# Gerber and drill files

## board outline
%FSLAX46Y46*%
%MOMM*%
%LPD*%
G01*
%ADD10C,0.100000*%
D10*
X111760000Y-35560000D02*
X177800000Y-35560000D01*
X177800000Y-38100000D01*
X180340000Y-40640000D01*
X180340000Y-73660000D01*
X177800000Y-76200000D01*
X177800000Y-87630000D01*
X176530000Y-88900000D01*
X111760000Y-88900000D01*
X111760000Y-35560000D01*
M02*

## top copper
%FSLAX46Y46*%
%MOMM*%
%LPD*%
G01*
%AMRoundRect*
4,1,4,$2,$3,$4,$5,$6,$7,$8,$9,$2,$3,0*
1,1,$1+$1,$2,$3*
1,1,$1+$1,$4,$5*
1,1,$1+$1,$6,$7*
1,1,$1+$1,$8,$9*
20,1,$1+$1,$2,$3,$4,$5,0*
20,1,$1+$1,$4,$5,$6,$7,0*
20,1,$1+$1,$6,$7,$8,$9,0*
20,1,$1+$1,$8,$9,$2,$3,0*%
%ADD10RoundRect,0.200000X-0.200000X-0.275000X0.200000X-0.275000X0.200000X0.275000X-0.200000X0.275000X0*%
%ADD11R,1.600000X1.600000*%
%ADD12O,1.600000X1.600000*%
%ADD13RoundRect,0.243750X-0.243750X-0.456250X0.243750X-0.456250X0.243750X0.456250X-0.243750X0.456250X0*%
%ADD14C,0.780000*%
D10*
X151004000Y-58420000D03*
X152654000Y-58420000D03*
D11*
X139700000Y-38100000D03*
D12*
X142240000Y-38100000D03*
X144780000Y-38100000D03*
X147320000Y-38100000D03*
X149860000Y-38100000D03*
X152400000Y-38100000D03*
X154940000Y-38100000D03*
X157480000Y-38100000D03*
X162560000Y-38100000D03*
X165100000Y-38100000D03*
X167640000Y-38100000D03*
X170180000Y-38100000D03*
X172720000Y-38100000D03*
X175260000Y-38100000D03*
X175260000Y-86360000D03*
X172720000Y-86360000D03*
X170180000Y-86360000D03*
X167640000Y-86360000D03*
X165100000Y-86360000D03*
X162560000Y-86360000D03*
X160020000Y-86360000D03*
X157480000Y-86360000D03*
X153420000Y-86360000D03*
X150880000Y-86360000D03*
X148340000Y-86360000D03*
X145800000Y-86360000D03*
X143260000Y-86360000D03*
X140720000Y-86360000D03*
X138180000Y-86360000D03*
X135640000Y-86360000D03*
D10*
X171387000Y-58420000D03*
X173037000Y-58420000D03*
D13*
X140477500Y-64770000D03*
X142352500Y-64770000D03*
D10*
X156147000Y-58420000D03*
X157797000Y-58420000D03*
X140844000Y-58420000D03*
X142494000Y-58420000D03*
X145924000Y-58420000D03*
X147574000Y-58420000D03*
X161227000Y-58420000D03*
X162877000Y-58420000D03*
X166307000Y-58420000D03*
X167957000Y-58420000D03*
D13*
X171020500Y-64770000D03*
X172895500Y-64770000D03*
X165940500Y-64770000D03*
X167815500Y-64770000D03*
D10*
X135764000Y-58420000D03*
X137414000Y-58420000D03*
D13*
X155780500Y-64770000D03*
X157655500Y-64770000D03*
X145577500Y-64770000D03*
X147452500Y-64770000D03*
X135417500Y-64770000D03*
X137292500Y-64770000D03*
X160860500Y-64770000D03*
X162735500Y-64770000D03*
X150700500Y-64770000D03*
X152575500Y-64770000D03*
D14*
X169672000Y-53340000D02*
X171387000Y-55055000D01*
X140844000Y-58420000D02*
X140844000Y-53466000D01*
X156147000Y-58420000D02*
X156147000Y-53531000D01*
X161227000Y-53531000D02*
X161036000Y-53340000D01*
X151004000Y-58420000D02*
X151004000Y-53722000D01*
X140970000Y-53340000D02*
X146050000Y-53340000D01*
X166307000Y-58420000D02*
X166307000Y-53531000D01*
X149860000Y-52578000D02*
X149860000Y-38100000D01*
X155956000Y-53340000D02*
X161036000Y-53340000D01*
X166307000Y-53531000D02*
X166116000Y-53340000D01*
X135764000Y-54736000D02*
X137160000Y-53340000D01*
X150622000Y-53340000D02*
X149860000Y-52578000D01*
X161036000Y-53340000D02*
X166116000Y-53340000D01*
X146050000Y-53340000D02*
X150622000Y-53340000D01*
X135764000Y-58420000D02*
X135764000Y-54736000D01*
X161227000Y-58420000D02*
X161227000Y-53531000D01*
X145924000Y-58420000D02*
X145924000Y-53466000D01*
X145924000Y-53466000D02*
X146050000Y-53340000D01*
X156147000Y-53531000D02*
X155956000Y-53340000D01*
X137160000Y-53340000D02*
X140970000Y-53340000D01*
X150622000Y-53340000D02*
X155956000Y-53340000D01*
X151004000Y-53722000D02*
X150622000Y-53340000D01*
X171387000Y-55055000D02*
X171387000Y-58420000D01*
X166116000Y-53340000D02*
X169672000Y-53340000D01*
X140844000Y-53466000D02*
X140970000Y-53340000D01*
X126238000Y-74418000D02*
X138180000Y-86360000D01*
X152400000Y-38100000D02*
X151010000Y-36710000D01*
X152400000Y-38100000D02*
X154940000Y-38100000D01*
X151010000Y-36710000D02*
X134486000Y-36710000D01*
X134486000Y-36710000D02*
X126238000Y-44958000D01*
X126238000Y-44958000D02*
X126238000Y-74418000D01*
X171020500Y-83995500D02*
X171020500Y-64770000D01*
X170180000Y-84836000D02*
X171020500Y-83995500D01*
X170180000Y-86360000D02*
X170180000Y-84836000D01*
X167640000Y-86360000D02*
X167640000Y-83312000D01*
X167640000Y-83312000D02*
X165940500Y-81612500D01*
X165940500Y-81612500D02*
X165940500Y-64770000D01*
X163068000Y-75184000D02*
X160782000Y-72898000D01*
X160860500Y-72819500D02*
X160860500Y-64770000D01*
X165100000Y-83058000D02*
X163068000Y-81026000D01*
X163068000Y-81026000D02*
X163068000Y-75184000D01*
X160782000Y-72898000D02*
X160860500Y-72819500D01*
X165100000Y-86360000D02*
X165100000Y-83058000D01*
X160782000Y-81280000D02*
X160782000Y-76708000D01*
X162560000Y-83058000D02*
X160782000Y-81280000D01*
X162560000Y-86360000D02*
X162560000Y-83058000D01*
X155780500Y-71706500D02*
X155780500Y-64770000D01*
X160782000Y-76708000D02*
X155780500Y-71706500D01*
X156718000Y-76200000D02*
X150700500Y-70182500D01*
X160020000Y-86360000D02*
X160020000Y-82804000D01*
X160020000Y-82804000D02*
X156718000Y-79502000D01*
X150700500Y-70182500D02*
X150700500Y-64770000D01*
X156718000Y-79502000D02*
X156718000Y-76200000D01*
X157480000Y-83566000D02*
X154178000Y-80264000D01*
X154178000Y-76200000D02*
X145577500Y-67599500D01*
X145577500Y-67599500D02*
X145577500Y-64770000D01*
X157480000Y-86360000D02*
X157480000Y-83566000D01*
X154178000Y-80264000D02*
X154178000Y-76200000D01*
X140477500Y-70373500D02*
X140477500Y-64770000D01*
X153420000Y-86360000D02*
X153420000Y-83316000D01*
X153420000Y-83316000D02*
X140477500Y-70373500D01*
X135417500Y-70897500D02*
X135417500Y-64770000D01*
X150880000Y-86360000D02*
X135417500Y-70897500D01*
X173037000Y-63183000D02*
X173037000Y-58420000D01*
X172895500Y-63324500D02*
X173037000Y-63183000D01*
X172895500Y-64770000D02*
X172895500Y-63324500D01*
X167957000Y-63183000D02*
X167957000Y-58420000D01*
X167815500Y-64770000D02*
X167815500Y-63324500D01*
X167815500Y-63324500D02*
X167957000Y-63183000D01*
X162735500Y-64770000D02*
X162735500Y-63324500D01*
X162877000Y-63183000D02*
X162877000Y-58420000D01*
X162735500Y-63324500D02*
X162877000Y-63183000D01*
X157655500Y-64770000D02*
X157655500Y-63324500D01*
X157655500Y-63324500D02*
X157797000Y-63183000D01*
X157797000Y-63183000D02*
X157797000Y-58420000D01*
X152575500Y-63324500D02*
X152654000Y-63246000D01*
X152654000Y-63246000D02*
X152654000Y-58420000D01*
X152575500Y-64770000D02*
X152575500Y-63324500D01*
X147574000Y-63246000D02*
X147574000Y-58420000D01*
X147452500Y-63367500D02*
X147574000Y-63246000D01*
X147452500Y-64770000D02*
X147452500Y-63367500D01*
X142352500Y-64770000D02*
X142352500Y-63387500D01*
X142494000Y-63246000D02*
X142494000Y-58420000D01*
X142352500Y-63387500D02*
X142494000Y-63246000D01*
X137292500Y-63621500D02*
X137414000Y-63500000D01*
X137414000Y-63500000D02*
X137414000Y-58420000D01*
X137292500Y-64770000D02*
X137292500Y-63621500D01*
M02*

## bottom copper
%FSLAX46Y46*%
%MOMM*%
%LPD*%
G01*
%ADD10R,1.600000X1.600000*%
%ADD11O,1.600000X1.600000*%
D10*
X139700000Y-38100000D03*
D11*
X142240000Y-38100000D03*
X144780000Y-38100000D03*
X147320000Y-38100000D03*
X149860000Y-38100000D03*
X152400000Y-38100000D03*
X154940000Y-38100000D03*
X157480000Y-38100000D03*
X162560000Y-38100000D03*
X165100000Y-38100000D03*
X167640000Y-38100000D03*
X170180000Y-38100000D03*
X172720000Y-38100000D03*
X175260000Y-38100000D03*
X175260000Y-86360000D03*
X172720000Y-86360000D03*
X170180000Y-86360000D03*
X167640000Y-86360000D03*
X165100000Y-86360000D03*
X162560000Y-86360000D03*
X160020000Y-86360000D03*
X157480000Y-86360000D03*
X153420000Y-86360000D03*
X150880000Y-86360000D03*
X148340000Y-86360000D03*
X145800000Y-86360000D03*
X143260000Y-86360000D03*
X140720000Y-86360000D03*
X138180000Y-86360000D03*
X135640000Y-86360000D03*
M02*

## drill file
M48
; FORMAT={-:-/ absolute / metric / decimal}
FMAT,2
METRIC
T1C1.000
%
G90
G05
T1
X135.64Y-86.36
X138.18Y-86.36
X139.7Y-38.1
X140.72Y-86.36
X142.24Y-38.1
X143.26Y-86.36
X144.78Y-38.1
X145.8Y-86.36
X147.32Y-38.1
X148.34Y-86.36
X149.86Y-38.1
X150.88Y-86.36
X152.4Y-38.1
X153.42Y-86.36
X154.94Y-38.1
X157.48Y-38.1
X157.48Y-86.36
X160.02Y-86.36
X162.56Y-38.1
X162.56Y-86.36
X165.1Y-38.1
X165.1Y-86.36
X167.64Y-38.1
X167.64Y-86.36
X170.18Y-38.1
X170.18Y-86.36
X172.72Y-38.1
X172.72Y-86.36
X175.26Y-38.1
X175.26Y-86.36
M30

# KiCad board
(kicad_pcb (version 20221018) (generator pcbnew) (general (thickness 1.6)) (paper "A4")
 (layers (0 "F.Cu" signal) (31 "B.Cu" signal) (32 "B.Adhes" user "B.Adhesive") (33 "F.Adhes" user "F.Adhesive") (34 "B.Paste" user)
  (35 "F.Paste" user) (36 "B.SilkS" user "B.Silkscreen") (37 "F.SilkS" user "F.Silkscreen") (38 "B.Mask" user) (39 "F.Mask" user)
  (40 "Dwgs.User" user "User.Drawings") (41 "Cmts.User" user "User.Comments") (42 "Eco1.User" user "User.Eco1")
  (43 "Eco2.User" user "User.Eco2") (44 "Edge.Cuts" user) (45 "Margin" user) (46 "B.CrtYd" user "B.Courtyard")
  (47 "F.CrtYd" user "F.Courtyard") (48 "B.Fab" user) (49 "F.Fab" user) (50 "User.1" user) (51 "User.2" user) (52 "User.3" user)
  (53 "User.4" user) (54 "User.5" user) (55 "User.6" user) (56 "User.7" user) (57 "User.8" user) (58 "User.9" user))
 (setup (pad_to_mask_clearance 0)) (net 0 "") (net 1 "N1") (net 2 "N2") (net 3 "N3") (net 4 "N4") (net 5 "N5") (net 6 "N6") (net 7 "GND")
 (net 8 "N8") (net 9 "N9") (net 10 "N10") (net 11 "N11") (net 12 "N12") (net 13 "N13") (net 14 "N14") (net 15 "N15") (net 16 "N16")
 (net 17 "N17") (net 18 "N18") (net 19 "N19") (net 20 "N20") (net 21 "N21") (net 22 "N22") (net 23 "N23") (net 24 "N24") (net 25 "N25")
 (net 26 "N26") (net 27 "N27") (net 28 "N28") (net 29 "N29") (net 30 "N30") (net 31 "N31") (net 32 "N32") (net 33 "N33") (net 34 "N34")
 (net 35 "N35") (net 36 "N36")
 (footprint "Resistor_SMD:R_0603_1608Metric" (layer "F.Cu") (at 151.829 58.42)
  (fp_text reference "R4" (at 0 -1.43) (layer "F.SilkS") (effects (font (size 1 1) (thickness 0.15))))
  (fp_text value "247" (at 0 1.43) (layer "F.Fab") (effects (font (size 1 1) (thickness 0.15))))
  (pad "1" smd roundrect (at -0.825 0) (size 0.8 0.95) (layers "F.Cu" "F.Paste" "F.Mask") (roundrect_rratio 0.25) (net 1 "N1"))
  (pad "2" smd roundrect (at 0.825 0) (size 0.8 0.95) (layers "F.Cu" "F.Paste" "F.Mask") (roundrect_rratio 0.25) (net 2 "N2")))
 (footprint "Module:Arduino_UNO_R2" (layer "F.Cu") (at 139.7 38.1)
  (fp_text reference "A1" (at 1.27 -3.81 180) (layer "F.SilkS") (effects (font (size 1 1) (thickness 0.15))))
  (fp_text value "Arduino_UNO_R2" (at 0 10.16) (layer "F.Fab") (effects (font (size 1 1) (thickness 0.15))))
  (pad "1" thru_hole rect (at 0 0 90) (size 1.6 1.6) (drill 1) (layers "*.Cu" "*.Mask") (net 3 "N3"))
  (pad "2" thru_hole oval (at 2.54 0 90) (size 1.6 1.6) (drill 1) (layers "*.Cu" "*.Mask") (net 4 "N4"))
  (pad "3" thru_hole oval (at 5.08 0 90) (size 1.6 1.6) (drill 1) (layers "*.Cu" "*.Mask") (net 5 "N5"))
  (pad "4" thru_hole oval (at 7.62 0 90) (size 1.6 1.6) (drill 1) (layers "*.Cu" "*.Mask") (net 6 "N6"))
  (pad "5" thru_hole oval (at 10.16 0 90) (size 1.6 1.6) (drill 1) (layers "*.Cu" "*.Mask") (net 1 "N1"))
  (pad "6" thru_hole oval (at 12.7 0 90) (size 1.6 1.6) (drill 1) (layers "*.Cu" "*.Mask") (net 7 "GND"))
  (pad "7" thru_hole oval (at 15.24 0 90) (size 1.6 1.6) (drill 1) (layers "*.Cu" "*.Mask") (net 7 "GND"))
  (pad "8" thru_hole oval (at 17.78 0 90) (size 1.6 1.6) (drill 1) (layers "*.Cu" "*.Mask") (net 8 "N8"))
  (pad "9" thru_hole oval (at 22.86 0 90) (size 1.6 1.6) (drill 1) (layers "*.Cu" "*.Mask") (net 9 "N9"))
  (pad "10" thru_hole oval (at 25.4 0 90) (size 1.6 1.6) (drill 1) (layers "*.Cu" "*.Mask") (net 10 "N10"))
  (pad "11" thru_hole oval (at 27.94 0 90) (size 1.6 1.6) (drill 1) (layers "*.Cu" "*.Mask") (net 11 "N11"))
  (pad "12" thru_hole oval (at 30.48 0 90) (size 1.6 1.6) (drill 1) (layers "*.Cu" "*.Mask") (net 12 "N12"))
  (pad "13" thru_hole oval (at 33.02 0 90) (size 1.6 1.6) (drill 1) (layers "*.Cu" "*.Mask") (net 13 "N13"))
  (pad "14" thru_hole oval (at 35.56 0 90) (size 1.6 1.6) (drill 1) (layers "*.Cu" "*.Mask") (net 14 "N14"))
  (pad "15" thru_hole oval (at 35.56 48.26 90) (size 1.6 1.6) (drill 1) (layers "*.Cu" "*.Mask") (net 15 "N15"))
  (pad "16" thru_hole oval (at 33.02 48.26 90) (size 1.6 1.6) (drill 1) (layers "*.Cu" "*.Mask") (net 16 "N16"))
  (pad "17" thru_hole oval (at 30.48 48.26 90) (size 1.6 1.6) (drill 1) (layers "*.Cu" "*.Mask") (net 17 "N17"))
  (pad "18" thru_hole oval (at 27.94 48.26 90) (size 1.6 1.6) (drill 1) (layers "*.Cu" "*.Mask") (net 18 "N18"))
  (pad "19" thru_hole oval (at 25.4 48.26 90) (size 1.6 1.6) (drill 1) (layers "*.Cu" "*.Mask") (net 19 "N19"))
  (pad "20" thru_hole oval (at 22.86 48.26 90) (size 1.6 1.6) (drill 1) (layers "*.Cu" "*.Mask") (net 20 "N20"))
  (pad "21" thru_hole oval (at 20.32 48.26 90) (size 1.6 1.6) (drill 1) (layers "*.Cu" "*.Mask") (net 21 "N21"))
  (pad "22" thru_hole oval (at 17.78 48.26 90) (size 1.6 1.6) (drill 1) (layers "*.Cu" "*.Mask") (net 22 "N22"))
  (pad "23" thru_hole oval (at 13.72 48.26 90) (size 1.6 1.6) (drill 1) (layers "*.Cu" "*.Mask") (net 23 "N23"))
  (pad "24" thru_hole oval (at 11.18 48.26 90) (size 1.6 1.6) (drill 1) (layers "*.Cu" "*.Mask") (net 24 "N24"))
  (pad "25" thru_hole oval (at 8.64 48.26 90) (size 1.6 1.6) (drill 1) (layers "*.Cu" "*.Mask") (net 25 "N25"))
  (pad "26" thru_hole oval (at 6.1 48.26 90) (size 1.6 1.6) (drill 1) (layers "*.Cu" "*.Mask") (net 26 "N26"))
  (pad "27" thru_hole oval (at 3.56 48.26 90) (size 1.6 1.6) (drill 1) (layers "*.Cu" "*.Mask") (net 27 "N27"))
  (pad "28" thru_hole oval (at 1.02 48.26 90) (size 1.6 1.6) (drill 1) (layers "*.Cu" "*.Mask") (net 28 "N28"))
  (pad "29" thru_hole oval (at -1.52 48.26 90) (size 1.6 1.6) (drill 1) (layers "*.Cu" "*.Mask") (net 7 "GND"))
  (pad "30" thru_hole oval (at -4.06 48.26 90) (size 1.6 1.6) (drill 1) (layers "*.Cu" "*.Mask") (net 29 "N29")))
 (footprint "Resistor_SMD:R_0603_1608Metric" (layer "F.Cu") (at 172.212 58.42)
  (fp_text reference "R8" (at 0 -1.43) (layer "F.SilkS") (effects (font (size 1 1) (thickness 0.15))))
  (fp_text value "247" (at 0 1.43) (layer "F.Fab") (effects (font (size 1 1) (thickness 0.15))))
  (pad "1" smd roundrect (at -0.825 0) (size 0.8 0.95) (layers "F.Cu" "F.Paste" "F.Mask") (roundrect_rratio 0.25) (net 1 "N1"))
  (pad "2" smd roundrect (at 0.825 0) (size 0.8 0.95) (layers "F.Cu" "F.Paste" "F.Mask") (roundrect_rratio 0.25) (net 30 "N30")))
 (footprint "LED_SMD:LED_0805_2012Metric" (layer "F.Cu") (at 141.415 64.77)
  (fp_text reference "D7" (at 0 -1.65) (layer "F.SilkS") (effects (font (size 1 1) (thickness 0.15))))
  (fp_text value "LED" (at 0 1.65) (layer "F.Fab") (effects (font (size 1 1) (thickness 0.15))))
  (pad "1" smd roundrect (at -0.9375 0) (size 0.975 1.4) (layers "F.Cu" "F.Paste" "F.Mask") (roundrect_rratio 0.25) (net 23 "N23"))
  (pad "2" smd roundrect (at 0.9375 0) (size 0.975 1.4) (layers "F.Cu" "F.Paste" "F.Mask") (roundrect_rratio 0.25) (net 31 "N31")))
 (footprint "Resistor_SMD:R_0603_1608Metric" (layer "F.Cu") (at 156.972 58.42)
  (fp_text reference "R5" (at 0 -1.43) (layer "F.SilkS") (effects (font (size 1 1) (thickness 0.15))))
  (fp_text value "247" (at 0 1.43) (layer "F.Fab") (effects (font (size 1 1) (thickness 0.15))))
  (pad "1" smd roundrect (at -0.825 0) (size 0.8 0.95) (layers "F.Cu" "F.Paste" "F.Mask") (roundrect_rratio 0.25) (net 1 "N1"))
  (pad "2" smd roundrect (at 0.825 0) (size 0.8 0.95) (layers "F.Cu" "F.Paste" "F.Mask") (roundrect_rratio 0.25) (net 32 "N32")))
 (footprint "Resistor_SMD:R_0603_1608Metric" (layer "F.Cu") (at 141.669 58.42)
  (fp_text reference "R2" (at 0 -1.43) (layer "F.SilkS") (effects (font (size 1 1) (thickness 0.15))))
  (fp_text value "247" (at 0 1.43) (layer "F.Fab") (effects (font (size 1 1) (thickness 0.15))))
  (pad "1" smd roundrect (at -0.825 0) (size 0.8 0.95) (layers "F.Cu" "F.Paste" "F.Mask") (roundrect_rratio 0.25) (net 1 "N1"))
  (pad "2" smd roundrect (at 0.825 0) (size 0.8 0.95) (layers "F.Cu" "F.Paste" "F.Mask") (roundrect_rratio 0.25) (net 31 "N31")))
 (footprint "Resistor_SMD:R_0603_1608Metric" (layer "F.Cu") (at 146.749 58.42)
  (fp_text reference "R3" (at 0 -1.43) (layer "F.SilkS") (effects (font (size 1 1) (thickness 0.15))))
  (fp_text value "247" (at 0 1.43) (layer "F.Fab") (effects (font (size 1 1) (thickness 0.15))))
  (pad "1" smd roundrect (at -0.825 0) (size 0.8 0.95) (layers "F.Cu" "F.Paste" "F.Mask") (roundrect_rratio 0.25) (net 1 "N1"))
  (pad "2" smd roundrect (at 0.825 0) (size 0.8 0.95) (layers "F.Cu" "F.Paste" "F.Mask") (roundrect_rratio 0.25) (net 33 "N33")))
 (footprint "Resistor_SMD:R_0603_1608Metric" (layer "F.Cu") (at 162.052 58.42)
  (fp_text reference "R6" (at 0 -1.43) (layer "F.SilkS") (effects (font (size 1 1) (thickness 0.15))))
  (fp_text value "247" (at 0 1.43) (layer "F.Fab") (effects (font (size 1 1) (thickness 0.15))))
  (pad "1" smd roundrect (at -0.825 0) (size 0.8 0.95) (layers "F.Cu" "F.Paste" "F.Mask") (roundrect_rratio 0.25) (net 1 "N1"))
  (pad "2" smd roundrect (at 0.825 0) (size 0.8 0.95) (layers "F.Cu" "F.Paste" "F.Mask") (roundrect_rratio 0.25) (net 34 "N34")))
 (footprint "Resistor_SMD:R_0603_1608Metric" (layer "F.Cu") (at 167.132 58.42)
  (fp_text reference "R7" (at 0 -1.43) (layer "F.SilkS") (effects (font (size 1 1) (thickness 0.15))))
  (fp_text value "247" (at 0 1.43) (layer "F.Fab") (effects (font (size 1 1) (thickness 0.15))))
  (pad "1" smd roundrect (at -0.825 0) (size 0.8 0.95) (layers "F.Cu" "F.Paste" "F.Mask") (roundrect_rratio 0.25) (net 1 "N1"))
  (pad "2" smd roundrect (at 0.825 0) (size 0.8 0.95) (layers "F.Cu" "F.Paste" "F.Mask") (roundrect_rratio 0.25) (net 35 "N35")))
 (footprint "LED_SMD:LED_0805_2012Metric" (layer "F.Cu") (at 171.958 64.77)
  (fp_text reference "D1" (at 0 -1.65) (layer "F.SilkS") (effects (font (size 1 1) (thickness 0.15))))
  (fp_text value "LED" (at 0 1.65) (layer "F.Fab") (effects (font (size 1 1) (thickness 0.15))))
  (pad "1" smd roundrect (at -0.9375 0) (size 0.975 1.4) (layers "F.Cu" "F.Paste" "F.Mask") (roundrect_rratio 0.25) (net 17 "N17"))
  (pad "2" smd roundrect (at 0.9375 0) (size 0.975 1.4) (layers "F.Cu" "F.Paste" "F.Mask") (roundrect_rratio 0.25) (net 30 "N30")))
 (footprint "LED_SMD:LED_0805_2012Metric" (layer "F.Cu") (at 166.878 64.77)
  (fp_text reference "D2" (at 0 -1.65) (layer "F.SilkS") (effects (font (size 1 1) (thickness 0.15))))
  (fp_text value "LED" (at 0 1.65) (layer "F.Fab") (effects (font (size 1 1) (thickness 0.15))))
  (pad "1" smd roundrect (at -0.9375 0) (size 0.975 1.4) (layers "F.Cu" "F.Paste" "F.Mask") (roundrect_rratio 0.25) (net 18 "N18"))
  (pad "2" smd roundrect (at 0.9375 0) (size 0.975 1.4) (layers "F.Cu" "F.Paste" "F.Mask") (roundrect_rratio 0.25) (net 35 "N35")))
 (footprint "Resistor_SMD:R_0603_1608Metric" (layer "F.Cu") (at 136.589 58.42)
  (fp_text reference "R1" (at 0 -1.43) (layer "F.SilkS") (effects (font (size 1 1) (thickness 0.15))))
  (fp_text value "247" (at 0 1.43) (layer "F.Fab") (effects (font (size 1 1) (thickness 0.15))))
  (pad "1" smd roundrect (at -0.825 0) (size 0.8 0.95) (layers "F.Cu" "F.Paste" "F.Mask") (roundrect_rratio 0.25) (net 1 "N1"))
  (pad "2" smd roundrect (at 0.825 0) (size 0.8 0.95) (layers "F.Cu" "F.Paste" "F.Mask") (roundrect_rratio 0.25) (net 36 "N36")))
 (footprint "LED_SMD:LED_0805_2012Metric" (layer "F.Cu") (at 156.718 64.77)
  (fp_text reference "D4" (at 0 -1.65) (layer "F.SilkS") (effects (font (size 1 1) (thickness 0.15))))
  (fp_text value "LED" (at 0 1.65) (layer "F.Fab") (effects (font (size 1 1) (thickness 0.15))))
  (pad "1" smd roundrect (at -0.9375 0) (size 0.975 1.4) (layers "F.Cu" "F.Paste" "F.Mask") (roundrect_rratio 0.25) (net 20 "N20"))
  (pad "2" smd roundrect (at 0.9375 0) (size 0.975 1.4) (layers "F.Cu" "F.Paste" "F.Mask") (roundrect_rratio 0.25) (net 32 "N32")))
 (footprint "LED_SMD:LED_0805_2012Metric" (layer "F.Cu") (at 146.515 64.77)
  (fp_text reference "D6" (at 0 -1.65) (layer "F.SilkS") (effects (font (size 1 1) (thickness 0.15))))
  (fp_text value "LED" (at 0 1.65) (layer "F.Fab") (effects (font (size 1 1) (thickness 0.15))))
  (pad "1" smd roundrect (at -0.9375 0) (size 0.975 1.4) (layers "F.Cu" "F.Paste" "F.Mask") (roundrect_rratio 0.25) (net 22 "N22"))
  (pad "2" smd roundrect (at 0.9375 0) (size 0.975 1.4) (layers "F.Cu" "F.Paste" "F.Mask") (roundrect_rratio 0.25) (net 33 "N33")))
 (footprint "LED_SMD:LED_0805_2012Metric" (layer "F.Cu") (at 136.355 64.77)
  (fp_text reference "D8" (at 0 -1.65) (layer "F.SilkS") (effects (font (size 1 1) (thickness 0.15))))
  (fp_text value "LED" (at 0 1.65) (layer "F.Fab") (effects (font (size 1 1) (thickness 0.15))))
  (pad "1" smd roundrect (at -0.9375 0) (size 0.975 1.4) (layers "F.Cu" "F.Paste" "F.Mask") (roundrect_rratio 0.25) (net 24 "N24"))
  (pad "2" smd roundrect (at 0.9375 0) (size 0.975 1.4) (layers "F.Cu" "F.Paste" "F.Mask") (roundrect_rratio 0.25) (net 36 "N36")))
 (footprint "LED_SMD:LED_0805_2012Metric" (layer "F.Cu") (at 161.798 64.77)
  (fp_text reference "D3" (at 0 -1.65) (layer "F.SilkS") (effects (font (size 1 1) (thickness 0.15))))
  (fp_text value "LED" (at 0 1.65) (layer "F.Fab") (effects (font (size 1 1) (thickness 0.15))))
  (pad "1" smd roundrect (at -0.9375 0) (size 0.975 1.4) (layers "F.Cu" "F.Paste" "F.Mask") (roundrect_rratio 0.25) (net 19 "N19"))
  (pad "2" smd roundrect (at 0.9375 0) (size 0.975 1.4) (layers "F.Cu" "F.Paste" "F.Mask") (roundrect_rratio 0.25) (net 34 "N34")))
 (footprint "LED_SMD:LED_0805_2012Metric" (layer "F.Cu") (at 151.638 64.77)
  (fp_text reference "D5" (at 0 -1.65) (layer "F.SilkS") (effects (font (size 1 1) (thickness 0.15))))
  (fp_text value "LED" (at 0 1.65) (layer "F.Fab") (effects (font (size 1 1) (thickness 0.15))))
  (pad "1" smd roundrect (at -0.9375 0) (size 0.975 1.4) (layers "F.Cu" "F.Paste" "F.Mask") (roundrect_rratio 0.25) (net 21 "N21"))
  (pad "2" smd roundrect (at 0.9375 0) (size 0.975 1.4) (layers "F.Cu" "F.Paste" "F.Mask") (roundrect_rratio 0.25) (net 2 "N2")))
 (gr_poly
  (pts (xy 111.76 35.56) (xy 177.8 35.56) (xy 177.8 38.1) (xy 180.34 40.64) (xy 180.34 73.66) (xy 177.8 76.2) (xy 177.8 87.63)
   (xy 176.53 88.9) (xy 111.76 88.9))
  (stroke (width 0.1) (type solid)) (fill none) (layer "Edge.Cuts"))
 (segment (start 169.672 53.34) (end 171.387 55.055) (width 0.78) (layer "F.Cu") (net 1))
 (segment (start 140.844 58.42) (end 140.844 53.466) (width 0.78) (layer "F.Cu") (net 1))
 (segment (start 156.147 58.42) (end 156.147 53.531) (width 0.78) (layer "F.Cu") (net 1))
 (segment (start 161.227 53.531) (end 161.036 53.34) (width 0.78) (layer "F.Cu") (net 1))
 (segment (start 151.004 58.42) (end 151.004 53.722) (width 0.78) (layer "F.Cu") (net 1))
 (segment (start 140.97 53.34) (end 146.05 53.34) (width 0.78) (layer "F.Cu") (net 1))
 (segment (start 166.307 58.42) (end 166.307 53.531) (width 0.78) (layer "F.Cu") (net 1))
 (segment (start 149.86 52.578) (end 149.86 38.1) (width 0.78) (layer "F.Cu") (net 1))
 (segment (start 155.956 53.34) (end 161.036 53.34) (width 0.78) (layer "F.Cu") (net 1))
 (segment (start 166.307 53.531) (end 166.116 53.34) (width 0.78) (layer "F.Cu") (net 1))
 (segment (start 135.764 54.736) (end 137.16 53.34) (width 0.78) (layer "F.Cu") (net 1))
 (segment (start 150.622 53.34) (end 149.86 52.578) (width 0.78) (layer "F.Cu") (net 1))
 (segment (start 161.036 53.34) (end 166.116 53.34) (width 0.78) (layer "F.Cu") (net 1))
 (segment (start 146.05 53.34) (end 150.622 53.34) (width 0.78) (layer "F.Cu") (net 1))
 (segment (start 135.764 58.42) (end 135.764 54.736) (width 0.78) (layer "F.Cu") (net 1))
 (segment (start 161.227 58.42) (end 161.227 53.531) (width 0.78) (layer "F.Cu") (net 1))
 (segment (start 145.924 58.42) (end 145.924 53.466) (width 0.78) (layer "F.Cu") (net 1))
 (segment (start 145.924 53.466) (end 146.05 53.34) (width 0.78) (layer "F.Cu") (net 1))
 (segment (start 156.147 53.531) (end 155.956 53.34) (width 0.78) (layer "F.Cu") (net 1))
 (segment (start 137.16 53.34) (end 140.97 53.34) (width 0.78) (layer "F.Cu") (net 1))
 (segment (start 150.622 53.34) (end 155.956 53.34) (width 0.78) (layer "F.Cu") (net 1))
 (segment (start 151.004 53.722) (end 150.622 53.34) (width 0.78) (layer "F.Cu") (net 1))
 (segment (start 171.387 55.055) (end 171.387 58.42) (width 0.78) (layer "F.Cu") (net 1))
 (segment (start 166.116 53.34) (end 169.672 53.34) (width 0.78) (layer "F.Cu") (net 1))
 (segment (start 140.844 53.466) (end 140.97 53.34) (width 0.78) (layer "F.Cu") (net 1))
 (segment (start 126.238 74.418) (end 138.18 86.36) (width 0.78) (layer "F.Cu") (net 7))
 (segment (start 152.4 38.1) (end 151.01 36.71) (width 0.78) (layer "F.Cu") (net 7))
 (segment (start 152.4 38.1) (end 154.94 38.1) (width 0.78) (layer "F.Cu") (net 7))
 (segment (start 151.01 36.71) (end 134.486 36.71) (width 0.78) (layer "F.Cu") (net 7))
 (segment (start 134.486 36.71) (end 126.238 44.958) (width 0.78) (layer "F.Cu") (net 7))
 (segment (start 126.238 44.958) (end 126.238 74.418) (width 0.78) (layer "F.Cu") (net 7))
 (segment (start 171.0205 83.9955) (end 171.0205 64.77) (width 0.78) (layer "F.Cu") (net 17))
 (segment (start 170.18 84.836) (end 171.0205 83.9955) (width 0.78) (layer "F.Cu") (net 17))
 (segment (start 170.18 86.36) (end 170.18 84.836) (width 0.78) (layer "F.Cu") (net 17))
 (segment (start 167.64 86.36) (end 167.64 83.312) (width 0.78) (layer "F.Cu") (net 18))
 (segment (start 167.64 83.312) (end 165.9405 81.6125) (width 0.78) (layer "F.Cu") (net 18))
 (segment (start 165.9405 81.6125) (end 165.9405 64.77) (width 0.78) (layer "F.Cu") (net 18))
 (segment (start 163.068 75.184) (end 160.782 72.898) (width 0.78) (layer "F.Cu") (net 19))
 (segment (start 160.8605 72.8195) (end 160.8605 64.77) (width 0.78) (layer "F.Cu") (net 19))
 (segment (start 165.1 83.058) (end 163.068 81.026) (width 0.78) (layer "F.Cu") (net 19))
 (segment (start 163.068 81.026) (end 163.068 75.184) (width 0.78) (layer "F.Cu") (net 19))
 (segment (start 160.782 72.898) (end 160.8605 72.8195) (width 0.78) (layer "F.Cu") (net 19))
 (segment (start 165.1 86.36) (end 165.1 83.058) (width 0.78) (layer "F.Cu") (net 19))
 (segment (start 160.782 81.28) (end 160.782 76.708) (width 0.78) (layer "F.Cu") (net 20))
 (segment (start 162.56 83.058) (end 160.782 81.28) (width 0.78) (layer "F.Cu") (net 20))
 (segment (start 162.56 86.36) (end 162.56 83.058) (width 0.78) (layer "F.Cu") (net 20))
 (segment (start 155.7805 71.7065) (end 155.7805 64.77) (width 0.78) (layer "F.Cu") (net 20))
 (segment (start 160.782 76.708) (end 155.7805 71.7065) (width 0.78) (layer "F.Cu") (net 20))
 (segment (start 156.718 76.2) (end 150.7005 70.1825) (width 0.78) (layer "F.Cu") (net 21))
 (segment (start 160.02 86.36) (end 160.02 82.804) (width 0.78) (layer "F.Cu") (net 21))
 (segment (start 160.02 82.804) (end 156.718 79.502) (width 0.78) (layer "F.Cu") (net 21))
 (segment (start 150.7005 70.1825) (end 150.7005 64.77) (width 0.78) (layer "F.Cu") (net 21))
 (segment (start 156.718 79.502) (end 156.718 76.2) (width 0.78) (layer "F.Cu") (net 21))
 (segment (start 157.48 83.566) (end 154.178 80.264) (width 0.78) (layer "F.Cu") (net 22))
 (segment (start 154.178 76.2) (end 145.5775 67.5995) (width 0.78) (layer "F.Cu") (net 22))
 (segment (start 145.5775 67.5995) (end 145.5775 64.77) (width 0.78) (layer "F.Cu") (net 22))
 (segment (start 157.48 86.36) (end 157.48 83.566) (width 0.78) (layer "F.Cu") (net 22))
 (segment (start 154.178 80.264) (end 154.178 76.2) (width 0.78) (layer "F.Cu") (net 22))
 (segment (start 140.4775 70.3735) (end 140.4775 64.77) (width 0.78) (layer "F.Cu") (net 23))
 (segment (start 153.42 86.36) (end 153.42 83.316) (width 0.78) (layer "F.Cu") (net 23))
 (segment (start 153.42 83.316) (end 140.4775 70.3735) (width 0.78) (layer "F.Cu") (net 23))
 (segment (start 135.4175 70.8975) (end 135.4175 64.77) (width 0.78) (layer "F.Cu") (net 24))
 (segment (start 150.88 86.36) (end 135.4175 70.8975) (width 0.78) (layer "F.Cu") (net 24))
 (segment (start 173.037 63.183) (end 173.037 58.42) (width 0.78) (layer "F.Cu") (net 30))
 (segment (start 172.8955 63.3245) (end 173.037 63.183) (width 0.78) (layer "F.Cu") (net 30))
 (segment (start 172.8955 64.77) (end 172.8955 63.3245) (width 0.78) (layer "F.Cu") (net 30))
 (segment (start 167.957 63.183) (end 167.957 58.42) (width 0.78) (layer "F.Cu") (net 35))
 (segment (start 167.8155 64.77) (end 167.8155 63.3245) (width 0.78) (layer "F.Cu") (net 35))
 (segment (start 167.8155 63.3245) (end 167.957 63.183) (width 0.78) (layer "F.Cu") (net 35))
 (segment (start 162.7355 64.77) (end 162.7355 63.3245) (width 0.78) (layer "F.Cu") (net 34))
 (segment (start 162.877 63.183) (end 162.877 58.42) (width 0.78) (layer "F.Cu") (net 34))
 (segment (start 162.7355 63.3245) (end 162.877 63.183) (width 0.78) (layer "F.Cu") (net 34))
 (segment (start 157.6555 64.77) (end 157.6555 63.3245) (width 0.78) (layer "F.Cu") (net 32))
 (segment (start 157.6555 63.3245) (end 157.797 63.183) (width 0.78) (layer "F.Cu") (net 32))
 (segment (start 157.797 63.183) (end 157.797 58.42) (width 0.78) (layer "F.Cu") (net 32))
 (segment (start 152.5755 63.3245) (end 152.654 63.246) (width 0.78) (layer "F.Cu") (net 2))
 (segment (start 152.654 63.246) (end 152.654 58.42) (width 0.78) (layer "F.Cu") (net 2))
 (segment (start 152.5755 64.77) (end 152.5755 63.3245) (width 0.78) (layer "F.Cu") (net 2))
 (segment (start 147.574 63.246) (end 147.574 58.42) (width 0.78) (layer "F.Cu") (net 33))
 (segment (start 147.4525 63.3675) (end 147.574 63.246) (width 0.78) (layer "F.Cu") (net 33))
 (segment (start 147.4525 64.77) (end 147.4525 63.3675) (width 0.78) (layer "F.Cu") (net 33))
 (segment (start 142.3525 64.77) (end 142.3525 63.3875) (width 0.78) (layer "F.Cu") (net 31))
 (segment (start 142.494 63.246) (end 142.494 58.42) (width 0.78) (layer "F.Cu") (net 31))
 (segment (start 142.3525 63.3875) (end 142.494 63.246) (width 0.78) (layer "F.Cu") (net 31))
 (segment (start 137.2925 63.6215) (end 137.414 63.5) (width 0.78) (layer "F.Cu") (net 36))
 (segment (start 137.414 63.5) (end 137.414 58.42) (width 0.78) (layer "F.Cu") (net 36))
 (segment (start 137.2925 64.77) (end 137.2925 63.6215) (width 0.78) (layer "F.Cu") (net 36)))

